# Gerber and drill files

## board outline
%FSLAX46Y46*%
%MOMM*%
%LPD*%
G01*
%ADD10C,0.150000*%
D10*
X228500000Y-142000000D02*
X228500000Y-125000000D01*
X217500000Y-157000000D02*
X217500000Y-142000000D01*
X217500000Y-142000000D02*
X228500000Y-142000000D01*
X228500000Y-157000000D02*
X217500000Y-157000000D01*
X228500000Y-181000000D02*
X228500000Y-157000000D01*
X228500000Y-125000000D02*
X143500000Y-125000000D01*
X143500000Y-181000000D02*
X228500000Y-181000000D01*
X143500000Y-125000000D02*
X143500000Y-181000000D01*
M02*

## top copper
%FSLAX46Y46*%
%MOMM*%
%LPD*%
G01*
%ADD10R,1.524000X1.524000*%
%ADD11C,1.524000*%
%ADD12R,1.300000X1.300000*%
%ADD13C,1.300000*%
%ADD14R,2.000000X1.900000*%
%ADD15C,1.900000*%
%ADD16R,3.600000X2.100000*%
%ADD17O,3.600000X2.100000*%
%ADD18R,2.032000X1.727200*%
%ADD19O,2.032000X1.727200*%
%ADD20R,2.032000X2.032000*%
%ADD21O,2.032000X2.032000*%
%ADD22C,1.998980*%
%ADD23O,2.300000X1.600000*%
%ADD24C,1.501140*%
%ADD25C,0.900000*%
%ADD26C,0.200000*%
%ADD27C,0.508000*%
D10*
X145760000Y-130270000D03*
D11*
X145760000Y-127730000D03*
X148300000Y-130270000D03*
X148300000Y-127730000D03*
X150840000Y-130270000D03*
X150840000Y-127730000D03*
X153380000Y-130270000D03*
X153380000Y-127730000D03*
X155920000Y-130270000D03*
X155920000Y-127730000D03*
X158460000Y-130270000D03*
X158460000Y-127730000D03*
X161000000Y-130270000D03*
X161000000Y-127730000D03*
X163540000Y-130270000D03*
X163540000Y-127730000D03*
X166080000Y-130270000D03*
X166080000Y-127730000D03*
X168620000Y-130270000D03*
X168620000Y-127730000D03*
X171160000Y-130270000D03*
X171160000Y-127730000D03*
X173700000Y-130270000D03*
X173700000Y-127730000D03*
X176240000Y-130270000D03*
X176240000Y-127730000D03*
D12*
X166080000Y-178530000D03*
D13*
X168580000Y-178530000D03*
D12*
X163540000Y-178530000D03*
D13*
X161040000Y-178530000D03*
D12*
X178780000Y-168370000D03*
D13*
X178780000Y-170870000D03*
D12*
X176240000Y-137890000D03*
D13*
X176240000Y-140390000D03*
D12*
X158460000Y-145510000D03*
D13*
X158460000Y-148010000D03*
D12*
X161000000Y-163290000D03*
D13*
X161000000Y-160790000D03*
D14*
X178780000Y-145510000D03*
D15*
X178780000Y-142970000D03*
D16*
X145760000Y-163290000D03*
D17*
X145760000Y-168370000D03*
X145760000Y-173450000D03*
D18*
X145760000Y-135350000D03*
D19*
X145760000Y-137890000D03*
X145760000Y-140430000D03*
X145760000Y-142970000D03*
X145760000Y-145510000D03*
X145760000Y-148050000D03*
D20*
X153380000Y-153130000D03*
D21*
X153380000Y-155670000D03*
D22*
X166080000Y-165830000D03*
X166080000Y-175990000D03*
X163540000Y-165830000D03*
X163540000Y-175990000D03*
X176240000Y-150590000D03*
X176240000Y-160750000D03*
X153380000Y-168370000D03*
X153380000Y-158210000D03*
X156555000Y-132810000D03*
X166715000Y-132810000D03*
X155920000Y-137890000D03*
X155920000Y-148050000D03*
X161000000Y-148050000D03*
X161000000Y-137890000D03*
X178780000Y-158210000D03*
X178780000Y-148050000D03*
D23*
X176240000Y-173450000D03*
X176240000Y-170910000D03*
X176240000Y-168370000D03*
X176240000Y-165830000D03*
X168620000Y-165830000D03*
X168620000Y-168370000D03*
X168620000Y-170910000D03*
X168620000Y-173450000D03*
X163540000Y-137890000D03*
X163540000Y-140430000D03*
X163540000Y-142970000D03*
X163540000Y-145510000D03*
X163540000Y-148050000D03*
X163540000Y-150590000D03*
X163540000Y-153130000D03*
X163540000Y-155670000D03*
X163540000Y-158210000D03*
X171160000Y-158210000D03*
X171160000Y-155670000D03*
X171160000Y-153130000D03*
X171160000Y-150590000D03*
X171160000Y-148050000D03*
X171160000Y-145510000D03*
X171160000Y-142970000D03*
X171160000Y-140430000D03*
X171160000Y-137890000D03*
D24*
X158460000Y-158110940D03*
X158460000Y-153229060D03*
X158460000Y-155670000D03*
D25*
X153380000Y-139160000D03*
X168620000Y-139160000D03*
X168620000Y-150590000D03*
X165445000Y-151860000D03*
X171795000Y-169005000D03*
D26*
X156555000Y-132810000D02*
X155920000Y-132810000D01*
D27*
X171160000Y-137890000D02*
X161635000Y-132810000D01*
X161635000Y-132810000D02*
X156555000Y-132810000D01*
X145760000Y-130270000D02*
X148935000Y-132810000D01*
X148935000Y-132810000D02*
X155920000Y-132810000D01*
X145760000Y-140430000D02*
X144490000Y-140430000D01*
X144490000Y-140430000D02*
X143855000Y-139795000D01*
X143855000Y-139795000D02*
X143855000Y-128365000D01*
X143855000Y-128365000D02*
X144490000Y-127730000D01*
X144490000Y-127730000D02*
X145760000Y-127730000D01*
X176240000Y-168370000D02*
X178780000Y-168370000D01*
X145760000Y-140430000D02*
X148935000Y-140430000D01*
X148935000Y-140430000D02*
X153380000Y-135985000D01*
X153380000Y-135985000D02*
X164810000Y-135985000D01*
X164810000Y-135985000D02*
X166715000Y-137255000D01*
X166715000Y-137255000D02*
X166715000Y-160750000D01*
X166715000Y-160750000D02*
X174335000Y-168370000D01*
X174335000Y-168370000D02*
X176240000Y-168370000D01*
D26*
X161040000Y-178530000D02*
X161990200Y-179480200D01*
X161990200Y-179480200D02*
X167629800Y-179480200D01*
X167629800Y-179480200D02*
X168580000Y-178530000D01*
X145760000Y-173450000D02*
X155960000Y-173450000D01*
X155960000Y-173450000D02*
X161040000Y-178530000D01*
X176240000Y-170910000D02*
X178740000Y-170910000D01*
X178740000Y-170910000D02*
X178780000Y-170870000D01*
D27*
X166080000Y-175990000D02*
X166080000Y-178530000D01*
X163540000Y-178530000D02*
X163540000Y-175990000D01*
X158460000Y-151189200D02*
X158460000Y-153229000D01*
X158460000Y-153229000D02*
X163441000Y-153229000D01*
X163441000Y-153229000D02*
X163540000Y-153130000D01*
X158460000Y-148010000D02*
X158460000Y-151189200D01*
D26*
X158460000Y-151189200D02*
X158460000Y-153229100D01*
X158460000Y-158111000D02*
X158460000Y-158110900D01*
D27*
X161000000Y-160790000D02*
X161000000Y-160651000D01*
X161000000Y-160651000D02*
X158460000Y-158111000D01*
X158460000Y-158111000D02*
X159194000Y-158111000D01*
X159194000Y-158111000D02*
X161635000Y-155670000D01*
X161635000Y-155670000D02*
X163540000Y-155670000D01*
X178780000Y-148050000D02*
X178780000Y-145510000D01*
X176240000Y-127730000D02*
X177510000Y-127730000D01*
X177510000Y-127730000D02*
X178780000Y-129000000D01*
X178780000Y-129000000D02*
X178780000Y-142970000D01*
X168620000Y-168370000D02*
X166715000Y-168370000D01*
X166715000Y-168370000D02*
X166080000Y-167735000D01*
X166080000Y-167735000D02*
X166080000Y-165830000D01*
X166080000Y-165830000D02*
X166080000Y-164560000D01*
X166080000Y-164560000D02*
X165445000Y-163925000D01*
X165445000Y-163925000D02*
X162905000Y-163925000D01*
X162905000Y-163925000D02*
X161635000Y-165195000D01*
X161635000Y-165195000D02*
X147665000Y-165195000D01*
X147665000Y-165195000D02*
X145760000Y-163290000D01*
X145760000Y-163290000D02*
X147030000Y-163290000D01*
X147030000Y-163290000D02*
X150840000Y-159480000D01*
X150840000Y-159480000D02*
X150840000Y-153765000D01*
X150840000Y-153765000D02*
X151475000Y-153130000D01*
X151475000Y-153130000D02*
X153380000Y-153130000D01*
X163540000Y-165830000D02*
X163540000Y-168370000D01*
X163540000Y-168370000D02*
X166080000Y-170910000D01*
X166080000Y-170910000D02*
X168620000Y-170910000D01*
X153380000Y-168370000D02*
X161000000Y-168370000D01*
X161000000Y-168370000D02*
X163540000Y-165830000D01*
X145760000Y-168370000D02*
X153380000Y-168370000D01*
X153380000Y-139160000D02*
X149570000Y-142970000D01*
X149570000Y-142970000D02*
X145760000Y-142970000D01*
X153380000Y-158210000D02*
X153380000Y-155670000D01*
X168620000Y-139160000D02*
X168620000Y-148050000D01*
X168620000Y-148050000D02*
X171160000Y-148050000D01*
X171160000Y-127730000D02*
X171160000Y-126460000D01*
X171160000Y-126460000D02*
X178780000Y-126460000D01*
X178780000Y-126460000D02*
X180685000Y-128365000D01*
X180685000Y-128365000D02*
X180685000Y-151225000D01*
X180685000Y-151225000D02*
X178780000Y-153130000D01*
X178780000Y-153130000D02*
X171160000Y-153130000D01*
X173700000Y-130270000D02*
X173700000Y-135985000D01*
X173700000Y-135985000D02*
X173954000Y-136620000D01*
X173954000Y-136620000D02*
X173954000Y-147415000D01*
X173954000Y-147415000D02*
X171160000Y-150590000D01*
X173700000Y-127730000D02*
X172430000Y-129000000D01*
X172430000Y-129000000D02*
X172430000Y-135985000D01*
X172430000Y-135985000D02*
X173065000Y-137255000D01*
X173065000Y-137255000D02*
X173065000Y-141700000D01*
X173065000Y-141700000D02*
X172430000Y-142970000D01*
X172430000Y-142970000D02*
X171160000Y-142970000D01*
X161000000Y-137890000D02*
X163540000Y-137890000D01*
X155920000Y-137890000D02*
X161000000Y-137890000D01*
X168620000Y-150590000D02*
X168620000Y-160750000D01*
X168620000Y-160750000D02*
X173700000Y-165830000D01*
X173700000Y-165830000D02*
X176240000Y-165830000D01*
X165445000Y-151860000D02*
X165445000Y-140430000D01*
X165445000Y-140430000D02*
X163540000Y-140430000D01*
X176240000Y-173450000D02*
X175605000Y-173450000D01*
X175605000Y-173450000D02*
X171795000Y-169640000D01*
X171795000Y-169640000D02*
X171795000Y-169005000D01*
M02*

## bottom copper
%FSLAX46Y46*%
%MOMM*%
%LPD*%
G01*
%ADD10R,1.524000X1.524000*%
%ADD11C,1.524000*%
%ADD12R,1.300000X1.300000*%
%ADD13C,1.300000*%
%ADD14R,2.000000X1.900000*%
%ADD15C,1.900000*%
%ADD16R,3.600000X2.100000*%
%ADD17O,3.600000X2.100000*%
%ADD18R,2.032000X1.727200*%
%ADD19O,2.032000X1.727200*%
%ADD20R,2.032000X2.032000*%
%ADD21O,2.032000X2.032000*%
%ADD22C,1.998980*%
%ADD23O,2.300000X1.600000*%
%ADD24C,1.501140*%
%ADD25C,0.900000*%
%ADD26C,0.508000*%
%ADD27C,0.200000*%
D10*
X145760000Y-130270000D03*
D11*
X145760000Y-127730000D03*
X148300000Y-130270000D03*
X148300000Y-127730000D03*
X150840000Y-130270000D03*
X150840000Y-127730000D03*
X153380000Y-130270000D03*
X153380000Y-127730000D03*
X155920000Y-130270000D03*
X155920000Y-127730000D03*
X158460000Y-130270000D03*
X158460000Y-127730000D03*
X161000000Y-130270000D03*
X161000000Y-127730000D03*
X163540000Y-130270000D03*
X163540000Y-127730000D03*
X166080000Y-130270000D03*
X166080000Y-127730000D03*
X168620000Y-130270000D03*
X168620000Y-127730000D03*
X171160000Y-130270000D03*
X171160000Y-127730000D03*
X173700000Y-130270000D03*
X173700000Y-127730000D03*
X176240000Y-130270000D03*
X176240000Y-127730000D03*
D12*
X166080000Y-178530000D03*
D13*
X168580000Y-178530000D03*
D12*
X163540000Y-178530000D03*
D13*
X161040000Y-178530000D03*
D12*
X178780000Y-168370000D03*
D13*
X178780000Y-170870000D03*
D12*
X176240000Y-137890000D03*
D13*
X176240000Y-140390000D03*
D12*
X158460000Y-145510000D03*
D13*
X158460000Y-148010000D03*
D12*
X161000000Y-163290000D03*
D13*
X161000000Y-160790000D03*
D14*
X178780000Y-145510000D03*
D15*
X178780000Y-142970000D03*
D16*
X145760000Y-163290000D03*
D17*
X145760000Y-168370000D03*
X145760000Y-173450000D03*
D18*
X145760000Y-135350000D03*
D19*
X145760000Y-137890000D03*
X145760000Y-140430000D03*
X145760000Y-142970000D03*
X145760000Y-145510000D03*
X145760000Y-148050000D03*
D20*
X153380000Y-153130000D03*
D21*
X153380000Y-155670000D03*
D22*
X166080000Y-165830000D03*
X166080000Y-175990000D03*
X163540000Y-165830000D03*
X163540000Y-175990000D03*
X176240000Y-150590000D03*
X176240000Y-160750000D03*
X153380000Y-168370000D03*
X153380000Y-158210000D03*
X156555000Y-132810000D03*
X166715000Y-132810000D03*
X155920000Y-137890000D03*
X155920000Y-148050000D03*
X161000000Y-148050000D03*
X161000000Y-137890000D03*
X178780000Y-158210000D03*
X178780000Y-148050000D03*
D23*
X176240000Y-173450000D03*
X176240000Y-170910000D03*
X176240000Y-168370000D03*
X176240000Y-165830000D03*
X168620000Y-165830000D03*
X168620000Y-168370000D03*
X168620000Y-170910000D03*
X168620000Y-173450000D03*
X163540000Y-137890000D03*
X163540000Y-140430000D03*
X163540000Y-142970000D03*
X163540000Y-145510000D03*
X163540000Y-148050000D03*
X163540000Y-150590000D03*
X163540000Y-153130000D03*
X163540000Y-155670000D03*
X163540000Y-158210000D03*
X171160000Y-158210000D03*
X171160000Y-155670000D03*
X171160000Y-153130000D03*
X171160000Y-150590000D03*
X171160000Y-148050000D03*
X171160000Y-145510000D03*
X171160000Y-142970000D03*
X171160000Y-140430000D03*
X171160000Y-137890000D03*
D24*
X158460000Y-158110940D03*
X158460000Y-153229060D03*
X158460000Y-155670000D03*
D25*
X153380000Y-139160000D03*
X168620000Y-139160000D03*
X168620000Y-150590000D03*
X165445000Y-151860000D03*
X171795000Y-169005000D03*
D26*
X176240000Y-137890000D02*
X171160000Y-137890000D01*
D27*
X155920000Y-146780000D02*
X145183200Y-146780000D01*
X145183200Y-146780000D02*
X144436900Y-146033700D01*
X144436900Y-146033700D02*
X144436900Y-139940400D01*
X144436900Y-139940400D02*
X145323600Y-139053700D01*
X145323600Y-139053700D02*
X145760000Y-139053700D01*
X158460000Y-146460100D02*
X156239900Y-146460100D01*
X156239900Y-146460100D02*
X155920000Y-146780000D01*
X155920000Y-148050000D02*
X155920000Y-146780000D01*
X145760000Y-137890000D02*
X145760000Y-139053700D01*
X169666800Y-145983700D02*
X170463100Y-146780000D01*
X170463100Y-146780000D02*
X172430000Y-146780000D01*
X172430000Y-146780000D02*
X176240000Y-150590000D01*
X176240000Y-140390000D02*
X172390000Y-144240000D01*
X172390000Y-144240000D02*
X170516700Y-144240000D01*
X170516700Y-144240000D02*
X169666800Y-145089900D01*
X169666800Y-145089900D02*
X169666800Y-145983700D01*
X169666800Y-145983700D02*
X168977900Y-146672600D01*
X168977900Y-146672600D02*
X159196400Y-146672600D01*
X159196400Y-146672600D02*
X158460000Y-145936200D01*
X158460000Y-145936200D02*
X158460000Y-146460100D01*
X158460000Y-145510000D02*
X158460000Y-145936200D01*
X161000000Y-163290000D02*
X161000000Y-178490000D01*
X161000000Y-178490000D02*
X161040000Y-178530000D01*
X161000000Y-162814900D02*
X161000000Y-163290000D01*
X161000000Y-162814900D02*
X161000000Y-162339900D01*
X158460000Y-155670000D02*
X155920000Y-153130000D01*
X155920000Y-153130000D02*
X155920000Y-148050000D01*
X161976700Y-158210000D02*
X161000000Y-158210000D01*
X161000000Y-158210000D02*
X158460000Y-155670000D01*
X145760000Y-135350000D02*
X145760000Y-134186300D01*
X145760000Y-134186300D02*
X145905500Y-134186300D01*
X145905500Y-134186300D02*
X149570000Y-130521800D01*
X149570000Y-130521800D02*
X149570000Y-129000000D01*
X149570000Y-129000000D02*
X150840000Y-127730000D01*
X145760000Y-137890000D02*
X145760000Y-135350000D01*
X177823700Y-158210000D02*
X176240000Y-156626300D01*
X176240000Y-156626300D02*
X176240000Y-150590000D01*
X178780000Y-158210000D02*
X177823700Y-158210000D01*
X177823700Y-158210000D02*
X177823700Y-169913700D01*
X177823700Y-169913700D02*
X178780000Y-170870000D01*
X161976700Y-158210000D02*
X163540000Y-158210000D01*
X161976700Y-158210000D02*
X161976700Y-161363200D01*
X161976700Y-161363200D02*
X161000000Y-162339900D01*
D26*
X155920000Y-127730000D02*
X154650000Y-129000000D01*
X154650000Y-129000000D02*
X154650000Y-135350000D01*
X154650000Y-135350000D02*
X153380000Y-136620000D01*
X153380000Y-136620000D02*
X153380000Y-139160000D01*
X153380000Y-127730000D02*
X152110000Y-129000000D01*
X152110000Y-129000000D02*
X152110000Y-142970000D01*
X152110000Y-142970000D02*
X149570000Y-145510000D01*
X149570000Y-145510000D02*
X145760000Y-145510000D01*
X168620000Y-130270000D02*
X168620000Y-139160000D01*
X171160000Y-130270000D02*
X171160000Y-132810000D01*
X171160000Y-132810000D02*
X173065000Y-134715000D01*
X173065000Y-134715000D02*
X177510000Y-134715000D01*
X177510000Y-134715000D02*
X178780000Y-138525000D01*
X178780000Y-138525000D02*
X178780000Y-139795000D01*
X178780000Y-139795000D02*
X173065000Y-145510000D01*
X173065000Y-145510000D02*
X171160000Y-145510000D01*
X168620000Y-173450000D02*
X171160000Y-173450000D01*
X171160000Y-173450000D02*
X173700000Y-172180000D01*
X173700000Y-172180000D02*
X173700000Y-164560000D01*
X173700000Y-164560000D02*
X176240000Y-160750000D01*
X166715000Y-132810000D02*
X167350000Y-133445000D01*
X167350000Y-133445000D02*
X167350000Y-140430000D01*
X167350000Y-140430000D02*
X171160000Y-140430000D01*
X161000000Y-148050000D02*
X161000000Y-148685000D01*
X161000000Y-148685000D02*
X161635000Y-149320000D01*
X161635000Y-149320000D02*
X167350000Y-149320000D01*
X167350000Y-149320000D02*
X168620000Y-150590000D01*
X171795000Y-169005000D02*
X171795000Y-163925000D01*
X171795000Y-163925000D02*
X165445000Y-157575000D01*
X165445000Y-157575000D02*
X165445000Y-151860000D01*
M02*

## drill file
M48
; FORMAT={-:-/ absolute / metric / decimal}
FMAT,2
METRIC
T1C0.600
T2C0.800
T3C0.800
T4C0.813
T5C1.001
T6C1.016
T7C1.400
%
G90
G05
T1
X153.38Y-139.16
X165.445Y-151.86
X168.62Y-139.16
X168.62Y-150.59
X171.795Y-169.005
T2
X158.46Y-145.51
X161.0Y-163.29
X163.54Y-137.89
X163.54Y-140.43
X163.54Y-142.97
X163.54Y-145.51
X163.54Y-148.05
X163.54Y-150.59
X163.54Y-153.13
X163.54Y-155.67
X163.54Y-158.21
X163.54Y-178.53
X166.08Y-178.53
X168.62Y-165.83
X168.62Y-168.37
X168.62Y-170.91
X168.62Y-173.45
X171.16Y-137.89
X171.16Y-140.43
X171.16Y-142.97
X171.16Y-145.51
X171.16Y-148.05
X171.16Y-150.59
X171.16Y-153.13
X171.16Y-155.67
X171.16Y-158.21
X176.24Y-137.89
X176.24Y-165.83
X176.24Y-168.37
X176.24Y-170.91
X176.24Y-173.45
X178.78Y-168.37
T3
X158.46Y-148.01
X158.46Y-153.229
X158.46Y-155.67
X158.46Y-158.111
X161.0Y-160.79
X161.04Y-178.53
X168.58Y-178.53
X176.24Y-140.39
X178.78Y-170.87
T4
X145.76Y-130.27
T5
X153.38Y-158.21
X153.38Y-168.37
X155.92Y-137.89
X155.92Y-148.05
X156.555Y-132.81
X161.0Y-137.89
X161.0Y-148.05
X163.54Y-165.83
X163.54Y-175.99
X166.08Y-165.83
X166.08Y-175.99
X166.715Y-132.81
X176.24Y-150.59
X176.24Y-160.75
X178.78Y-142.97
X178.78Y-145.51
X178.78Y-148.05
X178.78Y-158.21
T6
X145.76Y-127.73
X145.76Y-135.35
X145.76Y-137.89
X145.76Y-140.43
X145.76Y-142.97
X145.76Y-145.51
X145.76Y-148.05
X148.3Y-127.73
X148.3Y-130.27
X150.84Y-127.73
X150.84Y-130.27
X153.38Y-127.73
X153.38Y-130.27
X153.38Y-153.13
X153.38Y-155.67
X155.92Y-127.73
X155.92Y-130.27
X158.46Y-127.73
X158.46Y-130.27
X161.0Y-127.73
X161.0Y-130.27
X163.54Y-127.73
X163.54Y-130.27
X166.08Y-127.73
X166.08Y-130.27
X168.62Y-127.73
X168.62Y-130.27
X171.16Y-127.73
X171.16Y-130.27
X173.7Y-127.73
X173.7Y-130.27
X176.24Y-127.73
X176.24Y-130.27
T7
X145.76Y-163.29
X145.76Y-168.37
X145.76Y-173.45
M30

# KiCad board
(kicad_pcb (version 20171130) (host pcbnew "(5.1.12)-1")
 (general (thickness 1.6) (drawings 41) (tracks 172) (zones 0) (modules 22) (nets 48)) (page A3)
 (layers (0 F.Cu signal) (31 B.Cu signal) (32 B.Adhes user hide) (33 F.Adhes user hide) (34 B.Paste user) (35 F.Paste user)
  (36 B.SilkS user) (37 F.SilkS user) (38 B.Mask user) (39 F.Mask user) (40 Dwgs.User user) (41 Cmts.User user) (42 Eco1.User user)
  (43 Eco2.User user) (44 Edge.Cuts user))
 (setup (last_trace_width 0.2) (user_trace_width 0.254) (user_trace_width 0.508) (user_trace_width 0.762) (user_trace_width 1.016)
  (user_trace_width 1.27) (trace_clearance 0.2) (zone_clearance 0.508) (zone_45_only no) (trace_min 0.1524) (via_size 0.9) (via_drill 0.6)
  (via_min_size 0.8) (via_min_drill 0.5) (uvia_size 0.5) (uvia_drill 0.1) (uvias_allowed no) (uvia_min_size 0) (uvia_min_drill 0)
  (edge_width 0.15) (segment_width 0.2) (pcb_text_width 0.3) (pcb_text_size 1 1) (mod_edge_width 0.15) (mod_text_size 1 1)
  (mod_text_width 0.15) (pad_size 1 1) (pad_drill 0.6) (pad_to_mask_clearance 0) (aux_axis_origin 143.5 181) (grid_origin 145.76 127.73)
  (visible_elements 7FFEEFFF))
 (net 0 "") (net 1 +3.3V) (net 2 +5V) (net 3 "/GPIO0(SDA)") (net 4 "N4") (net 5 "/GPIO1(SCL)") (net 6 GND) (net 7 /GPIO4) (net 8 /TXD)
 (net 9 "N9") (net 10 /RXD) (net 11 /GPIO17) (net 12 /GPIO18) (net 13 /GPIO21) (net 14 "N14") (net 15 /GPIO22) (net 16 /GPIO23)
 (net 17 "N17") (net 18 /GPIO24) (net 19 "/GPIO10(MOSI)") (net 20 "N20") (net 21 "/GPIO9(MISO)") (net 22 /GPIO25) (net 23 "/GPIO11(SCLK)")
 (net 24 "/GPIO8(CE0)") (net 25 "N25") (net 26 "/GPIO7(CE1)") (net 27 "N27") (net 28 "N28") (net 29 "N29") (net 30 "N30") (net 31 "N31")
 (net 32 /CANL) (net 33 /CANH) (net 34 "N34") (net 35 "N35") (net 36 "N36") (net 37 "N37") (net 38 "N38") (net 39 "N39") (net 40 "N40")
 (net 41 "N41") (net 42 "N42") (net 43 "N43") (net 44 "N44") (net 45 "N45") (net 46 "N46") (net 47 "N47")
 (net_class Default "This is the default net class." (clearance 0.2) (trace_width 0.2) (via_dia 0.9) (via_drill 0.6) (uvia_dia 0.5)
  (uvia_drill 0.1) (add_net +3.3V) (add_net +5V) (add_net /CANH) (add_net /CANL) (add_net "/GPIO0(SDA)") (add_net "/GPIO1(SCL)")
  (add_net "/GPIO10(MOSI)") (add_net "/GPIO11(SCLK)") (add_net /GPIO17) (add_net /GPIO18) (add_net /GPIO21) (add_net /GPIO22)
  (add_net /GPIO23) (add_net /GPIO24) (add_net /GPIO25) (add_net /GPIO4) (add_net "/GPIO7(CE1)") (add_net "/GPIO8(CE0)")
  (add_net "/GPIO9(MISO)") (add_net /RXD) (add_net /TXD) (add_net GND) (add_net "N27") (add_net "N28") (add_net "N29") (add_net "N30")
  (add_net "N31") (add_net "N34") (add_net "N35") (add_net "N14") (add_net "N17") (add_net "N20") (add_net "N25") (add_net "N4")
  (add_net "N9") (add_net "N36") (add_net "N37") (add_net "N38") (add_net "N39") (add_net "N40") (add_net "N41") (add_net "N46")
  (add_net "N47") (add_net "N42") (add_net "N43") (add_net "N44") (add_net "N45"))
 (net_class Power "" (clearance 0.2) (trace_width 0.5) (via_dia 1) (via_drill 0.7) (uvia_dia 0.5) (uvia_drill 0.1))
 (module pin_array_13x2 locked (layer F.Cu) (at 161 129)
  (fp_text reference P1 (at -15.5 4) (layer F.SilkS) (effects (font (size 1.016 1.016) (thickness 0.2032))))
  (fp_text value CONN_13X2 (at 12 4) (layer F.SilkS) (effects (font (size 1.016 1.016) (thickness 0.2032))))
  (pad 1 thru_hole rect (at -15.24 1.27) (size 1.524 1.524) (drill 0.8128) (layers *.Cu *.Mask F.SilkS) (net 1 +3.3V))
  (pad 2 thru_hole circle (at -15.24 -1.27) (size 1.524 1.524) (drill 1.016) (layers *.Cu *.Mask F.SilkS) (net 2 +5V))
  (pad 3 thru_hole circle (at -12.7 1.27) (size 1.524 1.524) (drill 1.016) (layers *.Cu *.Mask F.SilkS) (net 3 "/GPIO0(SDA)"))
  (pad 4 thru_hole circle (at -12.7 -1.27) (size 1.524 1.524) (drill 1.016) (layers *.Cu *.Mask F.SilkS) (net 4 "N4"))
  (pad 5 thru_hole circle (at -10.16 1.27) (size 1.524 1.524) (drill 1.016) (layers *.Cu *.Mask F.SilkS) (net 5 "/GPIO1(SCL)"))
  (pad 6 thru_hole circle (at -10.16 -1.27) (size 1.524 1.524) (drill 1.016) (layers *.Cu *.Mask F.SilkS) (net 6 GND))
  (pad 7 thru_hole circle (at -7.62 1.27) (size 1.524 1.524) (drill 1.016) (layers *.Cu *.Mask F.SilkS) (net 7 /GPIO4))
  (pad 8 thru_hole circle (at -7.62 -1.27) (size 1.524 1.524) (drill 1.016) (layers *.Cu *.Mask F.SilkS) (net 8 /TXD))
  (pad 9 thru_hole circle (at -5.08 1.27) (size 1.524 1.524) (drill 1.016) (layers *.Cu *.Mask F.SilkS) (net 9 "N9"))
  (pad 10 thru_hole circle (at -5.08 -1.27) (size 1.524 1.524) (drill 1.016) (layers *.Cu *.Mask F.SilkS) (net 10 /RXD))
  (pad 11 thru_hole circle (at -2.54 1.27) (size 1.524 1.524) (drill 1.016) (layers *.Cu *.Mask F.SilkS) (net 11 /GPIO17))
  (pad 12 thru_hole circle (at -2.54 -1.27) (size 1.524 1.524) (drill 1.016) (layers *.Cu *.Mask F.SilkS) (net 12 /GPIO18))
  (pad 13 thru_hole circle (at 0 1.27) (size 1.524 1.524) (drill 1.016) (layers *.Cu *.Mask F.SilkS) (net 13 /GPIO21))
  (pad 14 thru_hole circle (at 0 -1.27) (size 1.524 1.524) (drill 1.016) (layers *.Cu *.Mask F.SilkS) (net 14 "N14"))
  (pad 15 thru_hole circle (at 2.54 1.27) (size 1.524 1.524) (drill 1.016) (layers *.Cu *.Mask F.SilkS) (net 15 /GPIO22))
  (pad 16 thru_hole circle (at 2.54 -1.27) (size 1.524 1.524) (drill 1.016) (layers *.Cu *.Mask F.SilkS) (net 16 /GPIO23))
  (pad 17 thru_hole circle (at 5.08 1.27) (size 1.524 1.524) (drill 1.016) (layers *.Cu *.Mask F.SilkS) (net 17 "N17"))
  (pad 18 thru_hole circle (at 5.08 -1.27) (size 1.524 1.524) (drill 1.016) (layers *.Cu *.Mask F.SilkS) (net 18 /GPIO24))
  (pad 19 thru_hole circle (at 7.62 1.27) (size 1.524 1.524) (drill 1.016) (layers *.Cu *.Mask F.SilkS) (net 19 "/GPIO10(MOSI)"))
  (pad 20 thru_hole circle (at 7.62 -1.27) (size 1.524 1.524) (drill 1.016) (layers *.Cu *.Mask F.SilkS) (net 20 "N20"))
  (pad 21 thru_hole circle (at 10.16 1.27) (size 1.524 1.524) (drill 1.016) (layers *.Cu *.Mask F.SilkS) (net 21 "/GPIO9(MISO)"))
  (pad 22 thru_hole circle (at 10.16 -1.27) (size 1.524 1.524) (drill 1.016) (layers *.Cu *.Mask F.SilkS) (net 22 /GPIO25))
  (pad 23 thru_hole circle (at 12.7 1.27) (size 1.524 1.524) (drill 1.016) (layers *.Cu *.Mask F.SilkS) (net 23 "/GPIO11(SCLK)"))
  (pad 24 thru_hole circle (at 12.7 -1.27) (size 1.524 1.524) (drill 1.016) (layers *.Cu *.Mask F.SilkS) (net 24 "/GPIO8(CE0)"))
  (pad 25 thru_hole circle (at 15.24 1.27) (size 1.524 1.524) (drill 1.016) (layers *.Cu *.Mask F.SilkS) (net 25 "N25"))
  (pad 26 thru_hole circle (at 15.24 -1.27) (size 1.524 1.524) (drill 1.016) (layers *.Cu *.Mask F.SilkS) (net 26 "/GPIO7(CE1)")))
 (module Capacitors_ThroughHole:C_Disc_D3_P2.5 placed (layer F.Cu) (at 166.08 178.53)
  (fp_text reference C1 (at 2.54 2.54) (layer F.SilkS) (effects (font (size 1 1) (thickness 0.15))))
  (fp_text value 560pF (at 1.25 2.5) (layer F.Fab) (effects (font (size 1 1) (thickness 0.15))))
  (pad 1 thru_hole rect (at 0 0) (size 1.3 1.3) (drill 0.8) (layers *.Cu *.Mask F.SilkS) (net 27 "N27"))
  (pad 2 thru_hole circle (at 2.5 0) (size 1.3 1.3) (drill 0.8001) (layers *.Cu *.Mask F.SilkS) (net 6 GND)))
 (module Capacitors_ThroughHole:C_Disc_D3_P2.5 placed (layer F.Cu) (at 163.54 178.53 180)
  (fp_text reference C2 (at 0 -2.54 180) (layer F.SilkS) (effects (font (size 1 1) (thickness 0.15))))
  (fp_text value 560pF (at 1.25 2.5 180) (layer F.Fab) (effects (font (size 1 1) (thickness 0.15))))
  (pad 1 thru_hole rect (at 0 0 180) (size 1.3 1.3) (drill 0.8) (layers *.Cu *.Mask F.SilkS) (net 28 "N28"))
  (pad 2 thru_hole circle (at 2.5 0 180) (size 1.3 1.3) (drill 0.8001) (layers *.Cu *.Mask F.SilkS) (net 6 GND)))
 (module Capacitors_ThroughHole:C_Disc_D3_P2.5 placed (layer F.Cu) (at 178.78 168.37 270)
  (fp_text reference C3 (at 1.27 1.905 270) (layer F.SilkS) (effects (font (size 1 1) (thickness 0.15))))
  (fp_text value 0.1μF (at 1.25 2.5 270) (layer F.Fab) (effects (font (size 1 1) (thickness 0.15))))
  (pad 1 thru_hole rect (at 0 0 270) (size 1.3 1.3) (drill 0.8) (layers *.Cu *.Mask F.SilkS) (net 2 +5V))
  (pad 2 thru_hole circle (at 2.5 0 270) (size 1.3 1.3) (drill 0.8001) (layers *.Cu *.Mask F.SilkS) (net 6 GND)))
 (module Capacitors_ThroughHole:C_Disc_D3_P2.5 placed (layer F.Cu) (at 176.24 137.89 270)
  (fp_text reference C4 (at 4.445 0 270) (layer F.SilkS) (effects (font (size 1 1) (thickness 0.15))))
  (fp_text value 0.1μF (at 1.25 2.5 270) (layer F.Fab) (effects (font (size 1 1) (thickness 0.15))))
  (pad 1 thru_hole rect (at 0 0 270) (size 1.3 1.3) (drill 0.8) (layers *.Cu *.Mask F.SilkS) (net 1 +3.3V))
  (pad 2 thru_hole circle (at 2.5 0 270) (size 1.3 1.3) (drill 0.8001) (layers *.Cu *.Mask F.SilkS) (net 6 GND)))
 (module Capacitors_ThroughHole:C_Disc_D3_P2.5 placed (layer F.Cu) (at 158.46 145.51 270)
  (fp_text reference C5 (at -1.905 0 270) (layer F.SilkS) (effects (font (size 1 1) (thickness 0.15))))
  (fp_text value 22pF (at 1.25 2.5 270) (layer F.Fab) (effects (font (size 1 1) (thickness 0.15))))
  (pad 1 thru_hole rect (at 0 0 270) (size 1.3 1.3) (drill 0.8) (layers *.Cu *.Mask F.SilkS) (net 6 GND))
  (pad 2 thru_hole circle (at 2.5 0 270) (size 1.3 1.3) (drill 0.8001) (layers *.Cu *.Mask F.SilkS) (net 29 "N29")))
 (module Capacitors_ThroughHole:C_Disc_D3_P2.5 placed (layer F.Cu) (at 161 163.29 90)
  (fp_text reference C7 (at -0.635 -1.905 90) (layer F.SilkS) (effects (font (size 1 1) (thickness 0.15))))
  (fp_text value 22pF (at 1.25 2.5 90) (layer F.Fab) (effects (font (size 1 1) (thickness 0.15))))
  (pad 1 thru_hole rect (at 0 0 90) (size 1.3 1.3) (drill 0.8) (layers *.Cu *.Mask F.SilkS) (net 6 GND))
  (pad 2 thru_hole circle (at 2.5 0 90) (size 1.3 1.3) (drill 0.8001) (layers *.Cu *.Mask F.SilkS) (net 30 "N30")))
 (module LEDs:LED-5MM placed (layer F.Cu) (at 178.78 145.51 90)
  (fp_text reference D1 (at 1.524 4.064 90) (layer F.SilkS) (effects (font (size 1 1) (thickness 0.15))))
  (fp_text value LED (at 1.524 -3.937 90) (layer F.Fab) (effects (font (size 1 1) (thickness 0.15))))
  (pad 1 thru_hole rect (at 0 0 180) (size 2 1.9) (drill 1.00076) (layers *.Cu *.Mask F.SilkS) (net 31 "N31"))
  (pad 2 thru_hole circle (at 2.54 0 90) (size 1.9 1.9) (drill 1.00076) (layers *.Cu *.Mask F.SilkS) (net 26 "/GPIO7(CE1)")))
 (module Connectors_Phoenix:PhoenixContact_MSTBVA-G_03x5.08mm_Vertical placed (layer F.Cu) (at 145.76 163.29 270)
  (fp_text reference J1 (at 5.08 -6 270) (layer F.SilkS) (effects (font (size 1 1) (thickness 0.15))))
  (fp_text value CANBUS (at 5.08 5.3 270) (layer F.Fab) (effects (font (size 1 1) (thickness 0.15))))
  (pad 1 thru_hole rect (at 0 0 270) (size 2.1 3.6) (drill 1.4) (layers *.Cu *.Mask) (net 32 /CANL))
  (pad 2 thru_hole oval (at 5.08 0 270) (size 2.1 3.6) (drill 1.4) (layers *.Cu *.Mask) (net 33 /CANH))
  (pad 3 thru_hole oval (at 10.16 0 270) (size 2.1 3.6) (drill 1.4) (layers *.Cu *.Mask) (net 6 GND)))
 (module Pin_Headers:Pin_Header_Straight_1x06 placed (layer F.Cu) (at 145.76 135.35)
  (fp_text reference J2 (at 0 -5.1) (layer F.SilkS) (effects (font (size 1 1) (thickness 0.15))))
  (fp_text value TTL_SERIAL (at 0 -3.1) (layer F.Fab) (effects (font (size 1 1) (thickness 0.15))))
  (pad 1 thru_hole rect (at 0 0) (size 2.032 1.7272) (drill 1.016) (layers *.Cu *.Mask F.SilkS) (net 6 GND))
  (pad 2 thru_hole oval (at 0 2.54) (size 2.032 1.7272) (drill 1.016) (layers *.Cu *.Mask F.SilkS) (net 6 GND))
  (pad 3 thru_hole oval (at 0 5.08) (size 2.032 1.7272) (drill 1.016) (layers *.Cu *.Mask F.SilkS) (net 2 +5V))
  (pad 4 thru_hole oval (at 0 7.62) (size 2.032 1.7272) (drill 1.016) (layers *.Cu *.Mask F.SilkS) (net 10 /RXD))
  (pad 5 thru_hole oval (at 0 10.16) (size 2.032 1.7272) (drill 1.016) (layers *.Cu *.Mask F.SilkS) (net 8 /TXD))
  (pad 6 thru_hole oval (at 0 12.7) (size 2.032 1.7272) (drill 1.016) (layers *.Cu *.Mask F.SilkS) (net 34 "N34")))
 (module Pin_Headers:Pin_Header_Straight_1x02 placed (layer F.Cu) (at 153.38 153.13)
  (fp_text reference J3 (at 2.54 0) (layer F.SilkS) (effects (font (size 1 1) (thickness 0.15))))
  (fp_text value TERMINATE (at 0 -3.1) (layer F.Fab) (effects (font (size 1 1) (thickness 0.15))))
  (pad 1 thru_hole rect (at 0 0) (size 2.032 2.032) (drill 1.016) (layers *.Cu *.Mask F.SilkS) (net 32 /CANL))
  (pad 2 thru_hole oval (at 0 2.54) (size 2.032 2.032) (drill 1.016) (layers *.Cu *.Mask F.SilkS) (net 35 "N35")))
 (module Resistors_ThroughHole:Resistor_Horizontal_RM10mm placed (layer F.Cu) (at 166.08 165.83 270)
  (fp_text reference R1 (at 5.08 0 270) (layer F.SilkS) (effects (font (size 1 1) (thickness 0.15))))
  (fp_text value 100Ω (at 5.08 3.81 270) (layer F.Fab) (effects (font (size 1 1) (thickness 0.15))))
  (pad 1 thru_hole circle (at 0 0 270) (size 1.99898 1.99898) (drill 1.00076) (layers *.Cu *.SilkS *.Mask) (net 32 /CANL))
  (pad 2 thru_hole circle (at 10.16 0 270) (size 1.99898 1.99898) (drill 1.00076) (layers *.Cu *.SilkS *.Mask) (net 27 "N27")))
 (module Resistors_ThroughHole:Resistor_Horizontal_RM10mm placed (layer F.Cu) (at 163.54 165.83 270)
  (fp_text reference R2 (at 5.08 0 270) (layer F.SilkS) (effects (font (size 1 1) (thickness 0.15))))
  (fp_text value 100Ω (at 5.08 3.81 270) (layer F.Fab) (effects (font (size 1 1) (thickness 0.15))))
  (pad 1 thru_hole circle (at 0 0 270) (size 1.99898 1.99898) (drill 1.00076) (layers *.Cu *.SilkS *.Mask) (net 33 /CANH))
  (pad 2 thru_hole circle (at 10.16 0 270) (size 1.99898 1.99898) (drill 1.00076) (layers *.Cu *.SilkS *.Mask) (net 28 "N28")))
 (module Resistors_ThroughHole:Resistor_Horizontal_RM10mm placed (layer F.Cu) (at 176.24 150.59 270)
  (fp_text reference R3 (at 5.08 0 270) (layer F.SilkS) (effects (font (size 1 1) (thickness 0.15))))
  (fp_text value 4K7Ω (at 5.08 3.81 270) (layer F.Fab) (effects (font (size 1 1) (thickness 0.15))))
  (pad 1 thru_hole circle (at 0 0 270) (size 1.99898 1.99898) (drill 1.00076) (layers *.Cu *.SilkS *.Mask) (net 6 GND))
  (pad 2 thru_hole circle (at 10.16 0 270) (size 1.99898 1.99898) (drill 1.00076) (layers *.Cu *.SilkS *.Mask) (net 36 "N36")))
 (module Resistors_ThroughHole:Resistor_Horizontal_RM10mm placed (layer F.Cu) (at 153.38 168.37 90)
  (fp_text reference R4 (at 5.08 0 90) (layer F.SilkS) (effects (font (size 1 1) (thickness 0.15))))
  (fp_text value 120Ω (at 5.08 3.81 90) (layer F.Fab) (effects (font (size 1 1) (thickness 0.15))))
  (pad 1 thru_hole circle (at 0 0 90) (size 1.99898 1.99898) (drill 1.00076) (layers *.Cu *.SilkS *.Mask) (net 33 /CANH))
  (pad 2 thru_hole circle (at 10.16 0 90) (size 1.99898 1.99898) (drill 1.00076) (layers *.Cu *.SilkS *.Mask) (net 35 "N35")))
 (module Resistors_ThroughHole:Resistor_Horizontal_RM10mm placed (layer F.Cu) (at 156.555 132.81)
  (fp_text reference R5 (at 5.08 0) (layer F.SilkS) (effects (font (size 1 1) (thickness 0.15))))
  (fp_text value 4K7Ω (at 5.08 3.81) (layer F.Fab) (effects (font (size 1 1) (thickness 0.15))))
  (pad 1 thru_hole circle (at 0 0) (size 1.99898 1.99898) (drill 1.00076) (layers *.Cu *.SilkS *.Mask) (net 1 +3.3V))
  (pad 2 thru_hole circle (at 10.16 0) (size 1.99898 1.99898) (drill 1.00076) (layers *.Cu *.SilkS *.Mask) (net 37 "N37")))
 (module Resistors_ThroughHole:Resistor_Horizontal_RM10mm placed (layer F.Cu) (at 155.92 137.89 270)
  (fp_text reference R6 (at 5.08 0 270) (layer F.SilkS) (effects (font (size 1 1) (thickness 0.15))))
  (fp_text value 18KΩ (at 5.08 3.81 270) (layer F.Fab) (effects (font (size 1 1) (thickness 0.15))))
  (pad 1 thru_hole circle (at 0 0 270) (size 1.99898 1.99898) (drill 1.00076) (layers *.Cu *.SilkS *.Mask) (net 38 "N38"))
  (pad 2 thru_hole circle (at 10.16 0 270) (size 1.99898 1.99898) (drill 1.00076) (layers *.Cu *.SilkS *.Mask) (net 6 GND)))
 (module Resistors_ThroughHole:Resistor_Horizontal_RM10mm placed (layer F.Cu) (at 161 148.05 90)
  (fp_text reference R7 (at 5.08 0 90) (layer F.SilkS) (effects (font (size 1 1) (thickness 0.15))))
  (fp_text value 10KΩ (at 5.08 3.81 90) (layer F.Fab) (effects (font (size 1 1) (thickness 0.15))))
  (pad 1 thru_hole circle (at 0 0 90) (size 1.99898 1.99898) (drill 1.00076) (layers *.Cu *.SilkS *.Mask) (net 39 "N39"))
  (pad 2 thru_hole circle (at 10.16 0 90) (size 1.99898 1.99898) (drill 1.00076) (layers *.Cu *.SilkS *.Mask) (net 38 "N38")))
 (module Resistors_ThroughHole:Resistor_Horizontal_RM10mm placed (layer F.Cu) (at 178.78 158.21 90)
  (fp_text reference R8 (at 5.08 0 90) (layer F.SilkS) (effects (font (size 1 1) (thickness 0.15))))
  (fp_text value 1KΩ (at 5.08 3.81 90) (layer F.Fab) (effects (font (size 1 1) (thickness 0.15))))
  (pad 1 thru_hole circle (at 0 0 90) (size 1.99898 1.99898) (drill 1.00076) (layers *.Cu *.SilkS *.Mask) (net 6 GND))
  (pad 2 thru_hole circle (at 10.16 0 90) (size 1.99898 1.99898) (drill 1.00076) (layers *.Cu *.SilkS *.Mask) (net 31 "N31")))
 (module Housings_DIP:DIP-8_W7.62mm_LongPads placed (layer F.Cu) (at 176.24 173.45 180)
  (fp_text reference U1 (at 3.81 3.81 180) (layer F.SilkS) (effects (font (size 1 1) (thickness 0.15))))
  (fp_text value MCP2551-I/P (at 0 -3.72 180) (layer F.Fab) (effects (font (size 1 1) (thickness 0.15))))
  (pad 1 thru_hole oval (at 0 0 180) (size 2.3 1.6) (drill 0.8) (layers *.Cu *.Mask F.SilkS) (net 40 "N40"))
  (pad 2 thru_hole oval (at 0 2.54 180) (size 2.3 1.6) (drill 0.8) (layers *.Cu *.Mask F.SilkS) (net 6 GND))
  (pad 3 thru_hole oval (at 0 5.08 180) (size 2.3 1.6) (drill 0.8) (layers *.Cu *.Mask F.SilkS) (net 2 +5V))
  (pad 4 thru_hole oval (at 0 7.62 180) (size 2.3 1.6) (drill 0.8) (layers *.Cu *.Mask F.SilkS) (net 39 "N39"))
  (pad 5 thru_hole oval (at 7.62 7.62 180) (size 2.3 1.6) (drill 0.8) (layers *.Cu *.Mask F.SilkS) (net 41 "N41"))
  (pad 6 thru_hole oval (at 7.62 5.08 180) (size 2.3 1.6) (drill 0.8) (layers *.Cu *.Mask F.SilkS) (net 32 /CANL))
  (pad 7 thru_hole oval (at 7.62 2.54 180) (size 2.3 1.6) (drill 0.8) (layers *.Cu *.Mask F.SilkS) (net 33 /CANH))
  (pad 8 thru_hole oval (at 7.62 0 180) (size 2.3 1.6) (drill 0.8) (layers *.Cu *.Mask F.SilkS) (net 36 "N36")))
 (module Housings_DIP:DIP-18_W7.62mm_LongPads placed (layer F.Cu) (at 163.54 137.89)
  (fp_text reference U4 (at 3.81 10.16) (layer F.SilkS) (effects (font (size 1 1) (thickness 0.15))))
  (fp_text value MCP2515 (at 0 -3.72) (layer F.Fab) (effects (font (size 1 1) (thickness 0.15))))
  (pad 1 thru_hole oval (at 0 0) (size 2.3 1.6) (drill 0.8) (layers *.Cu *.Mask F.SilkS) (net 38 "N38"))
  (pad 2 thru_hole oval (at 0 2.54) (size 2.3 1.6) (drill 0.8) (layers *.Cu *.Mask F.SilkS) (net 40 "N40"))
  (pad 3 thru_hole oval (at 0 5.08) (size 2.3 1.6) (drill 0.8) (layers *.Cu *.Mask F.SilkS) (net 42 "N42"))
  (pad 4 thru_hole oval (at 0 7.62) (size 2.3 1.6) (drill 0.8) (layers *.Cu *.Mask F.SilkS) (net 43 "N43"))
  (pad 5 thru_hole oval (at 0 10.16) (size 2.3 1.6) (drill 0.8) (layers *.Cu *.Mask F.SilkS) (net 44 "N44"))
  (pad 6 thru_hole oval (at 0 12.7) (size 2.3 1.6) (drill 0.8) (layers *.Cu *.Mask F.SilkS) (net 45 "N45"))
  (pad 7 thru_hole oval (at 0 15.24) (size 2.3 1.6) (drill 0.8) (layers *.Cu *.Mask F.SilkS) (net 29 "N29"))
  (pad 8 thru_hole oval (at 0 17.78) (size 2.3 1.6) (drill 0.8) (layers *.Cu *.Mask F.SilkS) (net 30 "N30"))
  (pad 9 thru_hole oval (at 0 20.32) (size 2.3 1.6) (drill 0.8) (layers *.Cu *.Mask F.SilkS) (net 6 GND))
  (pad 10 thru_hole oval (at 7.62 20.32) (size 2.3 1.6) (drill 0.8) (layers *.Cu *.Mask F.SilkS) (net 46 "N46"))
  (pad 11 thru_hole oval (at 7.62 17.78) (size 2.3 1.6) (drill 0.8) (layers *.Cu *.Mask F.SilkS) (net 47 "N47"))
  (pad 12 thru_hole oval (at 7.62 15.24) (size 2.3 1.6) (drill 0.8) (layers *.Cu *.Mask F.SilkS) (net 22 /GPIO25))
  (pad 13 thru_hole oval (at 7.62 12.7) (size 2.3 1.6) (drill 0.8) (layers *.Cu *.Mask F.SilkS) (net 23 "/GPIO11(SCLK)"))
  (pad 14 thru_hole oval (at 7.62 10.16) (size 2.3 1.6) (drill 0.8) (layers *.Cu *.Mask F.SilkS) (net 19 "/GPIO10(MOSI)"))
  (pad 15 thru_hole oval (at 7.62 7.62) (size 2.3 1.6) (drill 0.8) (layers *.Cu *.Mask F.SilkS) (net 21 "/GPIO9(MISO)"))
  (pad 16 thru_hole oval (at 7.62 5.08) (size 2.3 1.6) (drill 0.8) (layers *.Cu *.Mask F.SilkS) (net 24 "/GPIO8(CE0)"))
  (pad 17 thru_hole oval (at 7.62 2.54) (size 2.3 1.6) (drill 0.8) (layers *.Cu *.Mask F.SilkS) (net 37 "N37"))
  (pad 18 thru_hole oval (at 7.62 0) (size 2.3 1.6) (drill 0.8) (layers *.Cu *.Mask F.SilkS) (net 1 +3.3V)))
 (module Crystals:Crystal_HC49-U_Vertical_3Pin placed (layer F.Cu) (at 158.46 155.67 90)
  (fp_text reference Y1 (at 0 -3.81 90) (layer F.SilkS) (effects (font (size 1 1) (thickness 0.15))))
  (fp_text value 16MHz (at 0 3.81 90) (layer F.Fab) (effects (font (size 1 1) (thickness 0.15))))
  (pad 1 thru_hole circle (at -2.44094 0 90) (size 1.50114 1.50114) (drill 0.8001) (layers *.Cu *.Mask F.SilkS) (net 30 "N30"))
  (pad 2 thru_hole circle (at 2.44094 0 90) (size 1.50114 1.50114) (drill 0.8001) (layers *.Cu *.Mask F.SilkS) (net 29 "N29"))
  (pad 3 thru_hole circle (at 0 0 90) (size 1.50114 1.50114) (drill 0.8001) (layers *.Cu *.Mask F.SilkS) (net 6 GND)))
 (gr_line (start 228.5 142) (end 228.5 125) (angle 90) (layer Edge.Cuts) (width 0.15))
 (gr_line (start 217.5 157) (end 217.5 142) (angle 90) (layer Edge.Cuts) (width 0.15))
 (gr_line (start 217.5 142) (end 228.5 142) (angle 90) (layer Edge.Cuts) (width 0.15))
 (gr_line (start 228.5 157) (end 217.5 157) (angle 90) (layer Edge.Cuts) (width 0.15))
 (gr_line (start 228.5 181) (end 228.5 157) (angle 90) (layer Edge.Cuts) (width 0.15))
 (gr_line (start 228.5 125) (end 143.5 125) (angle 90) (layer Edge.Cuts) (width 0.15))
 (gr_line (start 143.5 181) (end 228.5 181) (angle 90) (layer Edge.Cuts) (width 0.15))
 (gr_line (start 143.5 125) (end 143.5 181) (angle 90) (layer Edge.Cuts) (width 0.15))
 (segment (start 156.555 132.81) (end 155.92 132.81) (width 0.2) (layer F.Cu) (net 1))
 (segment (start 171.16 137.89) (end 161.635 132.81) (width 0.508) (layer F.Cu) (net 1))
 (segment (start 161.635 132.81) (end 156.555 132.81) (width 0.508) (layer F.Cu) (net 1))
 (segment (start 145.76 130.27) (end 148.935 132.81) (width 0.508) (layer F.Cu) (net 1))
 (segment (start 148.935 132.81) (end 155.92 132.81) (width 0.508) (layer F.Cu) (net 1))
 (segment (start 176.24 137.89) (end 171.16 137.89) (width 0.508) (layer B.Cu) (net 1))
 (segment (start 145.76 140.43) (end 144.49 140.43) (width 0.508) (layer F.Cu) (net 2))
 (segment (start 144.49 140.43) (end 143.855 139.795) (width 0.508) (layer F.Cu) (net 2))
 (segment (start 143.855 139.795) (end 143.855 128.365) (width 0.508) (layer F.Cu) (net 2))
 (segment (start 143.855 128.365) (end 144.49 127.73) (width 0.508) (layer F.Cu) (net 2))
 (segment (start 144.49 127.73) (end 145.76 127.73) (width 0.508) (layer F.Cu) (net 2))
 (segment (start 176.24 168.37) (end 178.78 168.37) (width 0.508) (layer F.Cu) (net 2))
 (segment (start 145.76 140.43) (end 148.935 140.43) (width 0.508) (layer F.Cu) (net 2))
 (segment (start 148.935 140.43) (end 153.38 135.985) (width 0.508) (layer F.Cu) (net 2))
 (segment (start 153.38 135.985) (end 164.81 135.985) (width 0.508) (layer F.Cu) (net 2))
 (segment (start 164.81 135.985) (end 166.715 137.255) (width 0.508) (layer F.Cu) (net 2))
 (segment (start 166.715 137.255) (end 166.715 160.75) (width 0.508) (layer F.Cu) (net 2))
 (segment (start 166.715 160.75) (end 174.335 168.37) (width 0.508) (layer F.Cu) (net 2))
 (segment (start 174.335 168.37) (end 176.24 168.37) (width 0.508) (layer F.Cu) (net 2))
 (segment (start 155.92 146.78) (end 145.1832 146.78) (width 0.2) (layer B.Cu) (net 6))
 (segment (start 145.1832 146.78) (end 144.4369 146.0337) (width 0.2) (layer B.Cu) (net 6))
 (segment (start 144.4369 146.0337) (end 144.4369 139.9404) (width 0.2) (layer B.Cu) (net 6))
 (segment (start 144.4369 139.9404) (end 145.3236 139.0537) (width 0.2) (layer B.Cu) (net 6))
 (segment (start 145.3236 139.0537) (end 145.76 139.0537) (width 0.2) (layer B.Cu) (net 6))
 (segment (start 158.46 146.4601) (end 156.2399 146.4601) (width 0.2) (layer B.Cu) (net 6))
 (segment (start 156.2399 146.4601) (end 155.92 146.78) (width 0.2) (layer B.Cu) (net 6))
 (segment (start 155.92 148.05) (end 155.92 146.78) (width 0.2) (layer B.Cu) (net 6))
 (segment (start 145.76 137.89) (end 145.76 139.0537) (width 0.2) (layer B.Cu) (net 6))
 (segment (start 161.04 178.53) (end 161.9902 179.4802) (width 0.2) (layer F.Cu) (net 6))
 (segment (start 161.9902 179.4802) (end 167.6298 179.4802) (width 0.2) (layer F.Cu) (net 6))
 (segment (start 167.6298 179.4802) (end 168.58 178.53) (width 0.2) (layer F.Cu) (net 6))
 (segment (start 145.76 173.45) (end 155.96 173.45) (width 0.2) (layer F.Cu) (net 6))
 (segment (start 155.96 173.45) (end 161.04 178.53) (width 0.2) (layer F.Cu) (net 6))
 (segment (start 169.6668 145.9837) (end 170.4631 146.78) (width 0.2) (layer B.Cu) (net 6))
 (segment (start 170.4631 146.78) (end 172.43 146.78) (width 0.2) (layer B.Cu) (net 6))
 (segment (start 172.43 146.78) (end 176.24 150.59) (width 0.2) (layer B.Cu) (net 6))
 (segment (start 176.24 140.39) (end 172.39 144.24) (width 0.2) (layer B.Cu) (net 6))
 (segment (start 172.39 144.24) (end 170.5167 144.24) (width 0.2) (layer B.Cu) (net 6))
 (segment (start 170.5167 144.24) (end 169.6668 145.0899) (width 0.2) (layer B.Cu) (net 6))
 (segment (start 169.6668 145.0899) (end 169.6668 145.9837) (width 0.2) (layer B.Cu) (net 6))
 (segment (start 169.6668 145.9837) (end 168.9779 146.6726) (width 0.2) (layer B.Cu) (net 6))
 (segment (start 168.9779 146.6726) (end 159.1964 146.6726) (width 0.2) (layer B.Cu) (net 6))
 (segment (start 159.1964 146.6726) (end 158.46 145.9362) (width 0.2) (layer B.Cu) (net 6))
 (segment (start 158.46 145.9362) (end 158.46 146.4601) (width 0.2) (layer B.Cu) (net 6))
 (segment (start 158.46 145.51) (end 158.46 145.9362) (width 0.2) (layer B.Cu) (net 6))
 (segment (start 161 163.29) (end 161 178.49) (width 0.2) (layer B.Cu) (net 6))
 (segment (start 161 178.49) (end 161.04 178.53) (width 0.2) (layer B.Cu) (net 6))
 (segment (start 161 162.8149) (end 161 163.29) (width 0.2) (layer B.Cu) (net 6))
 (segment (start 161 162.8149) (end 161 162.3399) (width 0.2) (layer B.Cu) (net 6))
 (segment (start 158.46 155.67) (end 155.92 153.13) (width 0.2) (layer B.Cu) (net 6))
 (segment (start 155.92 153.13) (end 155.92 148.05) (width 0.2) (layer B.Cu) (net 6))
 (segment (start 161.9767 158.21) (end 161 158.21) (width 0.2) (layer B.Cu) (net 6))
 (segment (start 161 158.21) (end 158.46 155.67) (width 0.2) (layer B.Cu) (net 6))
 (segment (start 145.76 135.35) (end 145.76 134.1863) (width 0.2) (layer B.Cu) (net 6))
 (segment (start 145.76 134.1863) (end 145.9055 134.1863) (width 0.2) (layer B.Cu) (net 6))
 (segment (start 145.9055 134.1863) (end 149.57 130.5218) (width 0.2) (layer B.Cu) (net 6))
 (segment (start 149.57 130.5218) (end 149.57 129) (width 0.2) (layer B.Cu) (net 6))
 (segment (start 149.57 129) (end 150.84 127.73) (width 0.2) (layer B.Cu) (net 6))
 (segment (start 145.76 137.89) (end 145.76 135.35) (width 0.2) (layer B.Cu) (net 6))
 (segment (start 177.8237 158.21) (end 176.24 156.6263) (width 0.2) (layer B.Cu) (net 6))
 (segment (start 176.24 156.6263) (end 176.24 150.59) (width 0.2) (layer B.Cu) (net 6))
 (segment (start 178.78 158.21) (end 177.8237 158.21) (width 0.2) (layer B.Cu) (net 6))
 (segment (start 177.8237 158.21) (end 177.8237 169.9137) (width 0.2) (layer B.Cu) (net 6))
 (segment (start 177.8237 169.9137) (end 178.78 170.87) (width 0.2) (layer B.Cu) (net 6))
 (segment (start 176.24 170.91) (end 178.74 170.91) (width 0.2) (layer F.Cu) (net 6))
 (segment (start 178.74 170.91) (end 178.78 170.87) (width 0.2) (layer F.Cu) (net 6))
 (segment (start 161.9767 158.21) (end 163.54 158.21) (width 0.2) (layer B.Cu) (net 6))
 (segment (start 161.9767 158.21) (end 161.9767 161.3632) (width 0.2) (layer B.Cu) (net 6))
 (segment (start 161.9767 161.3632) (end 161 162.3399) (width 0.2) (layer B.Cu) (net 6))
 (segment (start 166.08 175.99) (end 166.08 178.53) (width 0.508) (layer F.Cu) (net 27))
 (segment (start 163.54 178.53) (end 163.54 175.99) (width 0.508) (layer F.Cu) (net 28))
 (segment (start 158.46 151.1892) (end 158.46 153.229) (width 0.508) (layer F.Cu) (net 29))
 (segment (start 158.46 153.229) (end 163.441 153.229) (width 0.508) (layer F.Cu) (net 29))
 (segment (start 163.441 153.229) (end 163.54 153.13) (width 0.508) (layer F.Cu) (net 29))
 (segment (start 158.46 148.01) (end 158.46 151.1892) (width 0.508) (layer F.Cu) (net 29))
 (segment (start 158.46 151.1892) (end 158.46 153.2291) (width 0.2) (layer F.Cu) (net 29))
 (segment (start 158.46 158.111) (end 158.46 158.1109) (width 0.2) (layer F.Cu) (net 30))
 (segment (start 161 160.79) (end 161 160.651) (width 0.508) (layer F.Cu) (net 30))
 (segment (start 161 160.651) (end 158.46 158.111) (width 0.508) (layer F.Cu) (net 30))
 (segment (start 158.46 158.111) (end 159.194 158.111) (width 0.508) (layer F.Cu) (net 30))
 (segment (start 159.194 158.111) (end 161.635 155.67) (width 0.508) (layer F.Cu) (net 30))
 (segment (start 161.635 155.67) (end 163.54 155.67) (width 0.508) (layer F.Cu) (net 30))
 (segment (start 178.78 148.05) (end 178.78 145.51) (width 0.508) (layer F.Cu) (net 31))
 (segment (start 176.24 127.73) (end 177.51 127.73) (width 0.508) (layer F.Cu) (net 26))
 (segment (start 177.51 127.73) (end 178.78 129) (width 0.508) (layer F.Cu) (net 26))
 (segment (start 178.78 129) (end 178.78 142.97) (width 0.508) (layer F.Cu) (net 26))
 (segment (start 168.62 168.37) (end 166.715 168.37) (width 0.508) (layer F.Cu) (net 32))
 (segment (start 166.715 168.37) (end 166.08 167.735) (width 0.508) (layer F.Cu) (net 32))
 (segment (start 166.08 167.735) (end 166.08 165.83) (width 0.508) (layer F.Cu) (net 32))
 (segment (start 166.08 165.83) (end 166.08 164.56) (width 0.508) (layer F.Cu) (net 32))
 (segment (start 166.08 164.56) (end 165.445 163.925) (width 0.508) (layer F.Cu) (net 32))
 (segment (start 165.445 163.925) (end 162.905 163.925) (width 0.508) (layer F.Cu) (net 32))
 (segment (start 162.905 163.925) (end 161.635 165.195) (width 0.508) (layer F.Cu) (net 32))
 (segment (start 161.635 165.195) (end 147.665 165.195) (width 0.508) (layer F.Cu) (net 32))
 (segment (start 147.665 165.195) (end 145.76 163.29) (width 0.508) (layer F.Cu) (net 32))
 (segment (start 145.76 163.29) (end 147.03 163.29) (width 0.508) (layer F.Cu) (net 32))
 (segment (start 147.03 163.29) (end 150.84 159.48) (width 0.508) (layer F.Cu) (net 32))
 (segment (start 150.84 159.48) (end 150.84 153.765) (width 0.508) (layer F.Cu) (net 32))
 (segment (start 150.84 153.765) (end 151.475 153.13) (width 0.508) (layer F.Cu) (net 32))
 (segment (start 151.475 153.13) (end 153.38 153.13) (width 0.508) (layer F.Cu) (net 32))
 (segment (start 163.54 165.83) (end 163.54 168.37) (width 0.508) (layer F.Cu) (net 33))
 (segment (start 163.54 168.37) (end 166.08 170.91) (width 0.508) (layer F.Cu) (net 33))
 (segment (start 166.08 170.91) (end 168.62 170.91) (width 0.508) (layer F.Cu) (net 33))
 (segment (start 153.38 168.37) (end 161 168.37) (width 0.508) (layer F.Cu) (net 33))
 (segment (start 161 168.37) (end 163.54 165.83) (width 0.508) (layer F.Cu) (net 33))
 (segment (start 145.76 168.37) (end 153.38 168.37) (width 0.508) (layer F.Cu) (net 33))
 (segment (start 155.92 127.73) (end 154.65 129) (width 0.508) (layer B.Cu) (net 10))
 (segment (start 154.65 129) (end 154.65 135.35) (width 0.508) (layer B.Cu) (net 10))
 (segment (start 154.65 135.35) (end 153.38 136.62) (width 0.508) (layer B.Cu) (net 10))
 (segment (start 153.38 136.62) (end 153.38 139.16) (width 0.508) (layer B.Cu) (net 10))
 (segment (start 153.38 139.16) (end 149.57 142.97) (width 0.508) (layer F.Cu) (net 10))
 (segment (start 149.57 142.97) (end 145.76 142.97) (width 0.508) (layer F.Cu) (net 10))
 (via (at 153.38 139.16) (size 0.9) (layers F.Cu B.Cu) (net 10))
 (segment (start 153.38 127.73) (end 152.11 129) (width 0.508) (layer B.Cu) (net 8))
 (segment (start 152.11 129) (end 152.11 142.97) (width 0.508) (layer B.Cu) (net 8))
 (segment (start 152.11 142.97) (end 149.57 145.51) (width 0.508) (layer B.Cu) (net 8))
 (segment (start 149.57 145.51) (end 145.76 145.51) (width 0.508) (layer B.Cu) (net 8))
 (segment (start 153.38 158.21) (end 153.38 155.67) (width 0.508) (layer F.Cu) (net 35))
 (segment (start 168.62 139.16) (end 168.62 148.05) (width 0.508) (layer F.Cu) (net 19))
 (segment (start 168.62 148.05) (end 171.16 148.05) (width 0.508) (layer F.Cu) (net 19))
 (segment (start 168.62 130.27) (end 168.62 139.16) (width 0.508) (layer B.Cu) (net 19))
 (via (at 168.62 139.16) (size 0.9) (layers F.Cu B.Cu) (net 19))
 (segment (start 171.16 130.27) (end 171.16 132.81) (width 0.508) (layer B.Cu) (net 21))
 (segment (start 171.16 132.81) (end 173.065 134.715) (width 0.508) (layer B.Cu) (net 21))
 (segment (start 173.065 134.715) (end 177.51 134.715) (width 0.508) (layer B.Cu) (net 21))
 (segment (start 177.51 134.715) (end 178.78 138.525) (width 0.508) (layer B.Cu) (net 21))
 (segment (start 178.78 138.525) (end 178.78 139.795) (width 0.508) (layer B.Cu) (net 21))
 (segment (start 178.78 139.795) (end 173.065 145.51) (width 0.508) (layer B.Cu) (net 21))
 (segment (start 173.065 145.51) (end 171.16 145.51) (width 0.508) (layer B.Cu) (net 21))
 (segment (start 171.16 127.73) (end 171.16 126.46) (width 0.508) (layer F.Cu) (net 22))
 (segment (start 171.16 126.46) (end 178.78 126.46) (width 0.508) (layer F.Cu) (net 22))
 (segment (start 178.78 126.46) (end 180.685 128.365) (width 0.508) (layer F.Cu) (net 22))
 (segment (start 180.685 128.365) (end 180.685 151.225) (width 0.508) (layer F.Cu) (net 22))
 (segment (start 180.685 151.225) (end 178.78 153.13) (width 0.508) (layer F.Cu) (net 22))
 (segment (start 178.78 153.13) (end 171.16 153.13) (width 0.508) (layer F.Cu) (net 22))
 (segment (start 173.7 130.27) (end 173.7 135.985) (width 0.508) (layer F.Cu) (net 23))
 (segment (start 173.7 135.985) (end 173.954 136.62) (width 0.508) (layer F.Cu) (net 23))
 (segment (start 173.954 136.62) (end 173.954 147.415) (width 0.508) (layer F.Cu) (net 23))
 (segment (start 173.954 147.415) (end 171.16 150.59) (width 0.508) (layer F.Cu) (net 23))
 (segment (start 173.7 127.73) (end 172.43 129) (width 0.508) (layer F.Cu) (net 24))
 (segment (start 172.43 129) (end 172.43 135.985) (width 0.508) (layer F.Cu) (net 24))
 (segment (start 172.43 135.985) (end 173.065 137.255) (width 0.508) (layer F.Cu) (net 24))
 (segment (start 173.065 137.255) (end 173.065 141.7) (width 0.508) (layer F.Cu) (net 24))
 (segment (start 173.065 141.7) (end 172.43 142.97) (width 0.508) (layer F.Cu) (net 24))
 (segment (start 172.43 142.97) (end 171.16 142.97) (width 0.508) (layer F.Cu) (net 24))
 (segment (start 168.62 173.45) (end 171.16 173.45) (width 0.508) (layer B.Cu) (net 36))
 (segment (start 171.16 173.45) (end 173.7 172.18) (width 0.508) (layer B.Cu) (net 36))
 (segment (start 173.7 172.18) (end 173.7 164.56) (width 0.508) (layer B.Cu) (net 36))
 (segment (start 173.7 164.56) (end 176.24 160.75) (width 0.508) (layer B.Cu) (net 36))
 (segment (start 166.715 132.81) (end 167.35 133.445) (width 0.508) (layer B.Cu) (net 37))
 (segment (start 167.35 133.445) (end 167.35 140.43) (width 0.508) (layer B.Cu) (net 37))
 (segment (start 167.35 140.43) (end 171.16 140.43) (width 0.508) (layer B.Cu) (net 37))
 (segment (start 161 137.89) (end 163.54 137.89) (width 0.508) (layer F.Cu) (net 38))
 (segment (start 155.92 137.89) (end 161 137.89) (width 0.508) (layer F.Cu) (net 38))
 (segment (start 168.62 150.59) (end 168.62 160.75) (width 0.508) (layer F.Cu) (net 39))
 (segment (start 168.62 160.75) (end 173.7 165.83) (width 0.508) (layer F.Cu) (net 39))
 (segment (start 173.7 165.83) (end 176.24 165.83) (width 0.508) (layer F.Cu) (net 39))
 (segment (start 161 148.05) (end 161 148.685) (width 0.508) (layer B.Cu) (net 39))
 (segment (start 161 148.685) (end 161.635 149.32) (width 0.508) (layer B.Cu) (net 39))
 (segment (start 161.635 149.32) (end 167.35 149.32) (width 0.508) (layer B.Cu) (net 39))
 (segment (start 167.35 149.32) (end 168.62 150.59) (width 0.508) (layer B.Cu) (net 39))
 (via (at 168.62 150.59) (size 0.9) (layers F.Cu B.Cu) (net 39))
 (segment (start 165.445 151.86) (end 165.445 140.43) (width 0.508) (layer F.Cu) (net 40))
 (segment (start 165.445 140.43) (end 163.54 140.43) (width 0.508) (layer F.Cu) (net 40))
 (segment (start 171.795 169.005) (end 171.795 163.925) (width 0.508) (layer B.Cu) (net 40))
 (segment (start 171.795 163.925) (end 165.445 157.575) (width 0.508) (layer B.Cu) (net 40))
 (segment (start 165.445 157.575) (end 165.445 151.86) (width 0.508) (layer B.Cu) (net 40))
 (segment (start 176.24 173.45) (end 175.605 173.45) (width 0.508) (layer F.Cu) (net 40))
 (segment (start 175.605 173.45) (end 171.795 169.64) (width 0.508) (layer F.Cu) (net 40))
 (segment (start 171.795 169.64) (end 171.795 169.005) (width 0.508) (layer F.Cu) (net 40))
 (via (at 165.445 151.86) (size 0.9) (layers F.Cu B.Cu) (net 40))
 (via (at 171.795 169.005) (size 0.9) (layers F.Cu B.Cu) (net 40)))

